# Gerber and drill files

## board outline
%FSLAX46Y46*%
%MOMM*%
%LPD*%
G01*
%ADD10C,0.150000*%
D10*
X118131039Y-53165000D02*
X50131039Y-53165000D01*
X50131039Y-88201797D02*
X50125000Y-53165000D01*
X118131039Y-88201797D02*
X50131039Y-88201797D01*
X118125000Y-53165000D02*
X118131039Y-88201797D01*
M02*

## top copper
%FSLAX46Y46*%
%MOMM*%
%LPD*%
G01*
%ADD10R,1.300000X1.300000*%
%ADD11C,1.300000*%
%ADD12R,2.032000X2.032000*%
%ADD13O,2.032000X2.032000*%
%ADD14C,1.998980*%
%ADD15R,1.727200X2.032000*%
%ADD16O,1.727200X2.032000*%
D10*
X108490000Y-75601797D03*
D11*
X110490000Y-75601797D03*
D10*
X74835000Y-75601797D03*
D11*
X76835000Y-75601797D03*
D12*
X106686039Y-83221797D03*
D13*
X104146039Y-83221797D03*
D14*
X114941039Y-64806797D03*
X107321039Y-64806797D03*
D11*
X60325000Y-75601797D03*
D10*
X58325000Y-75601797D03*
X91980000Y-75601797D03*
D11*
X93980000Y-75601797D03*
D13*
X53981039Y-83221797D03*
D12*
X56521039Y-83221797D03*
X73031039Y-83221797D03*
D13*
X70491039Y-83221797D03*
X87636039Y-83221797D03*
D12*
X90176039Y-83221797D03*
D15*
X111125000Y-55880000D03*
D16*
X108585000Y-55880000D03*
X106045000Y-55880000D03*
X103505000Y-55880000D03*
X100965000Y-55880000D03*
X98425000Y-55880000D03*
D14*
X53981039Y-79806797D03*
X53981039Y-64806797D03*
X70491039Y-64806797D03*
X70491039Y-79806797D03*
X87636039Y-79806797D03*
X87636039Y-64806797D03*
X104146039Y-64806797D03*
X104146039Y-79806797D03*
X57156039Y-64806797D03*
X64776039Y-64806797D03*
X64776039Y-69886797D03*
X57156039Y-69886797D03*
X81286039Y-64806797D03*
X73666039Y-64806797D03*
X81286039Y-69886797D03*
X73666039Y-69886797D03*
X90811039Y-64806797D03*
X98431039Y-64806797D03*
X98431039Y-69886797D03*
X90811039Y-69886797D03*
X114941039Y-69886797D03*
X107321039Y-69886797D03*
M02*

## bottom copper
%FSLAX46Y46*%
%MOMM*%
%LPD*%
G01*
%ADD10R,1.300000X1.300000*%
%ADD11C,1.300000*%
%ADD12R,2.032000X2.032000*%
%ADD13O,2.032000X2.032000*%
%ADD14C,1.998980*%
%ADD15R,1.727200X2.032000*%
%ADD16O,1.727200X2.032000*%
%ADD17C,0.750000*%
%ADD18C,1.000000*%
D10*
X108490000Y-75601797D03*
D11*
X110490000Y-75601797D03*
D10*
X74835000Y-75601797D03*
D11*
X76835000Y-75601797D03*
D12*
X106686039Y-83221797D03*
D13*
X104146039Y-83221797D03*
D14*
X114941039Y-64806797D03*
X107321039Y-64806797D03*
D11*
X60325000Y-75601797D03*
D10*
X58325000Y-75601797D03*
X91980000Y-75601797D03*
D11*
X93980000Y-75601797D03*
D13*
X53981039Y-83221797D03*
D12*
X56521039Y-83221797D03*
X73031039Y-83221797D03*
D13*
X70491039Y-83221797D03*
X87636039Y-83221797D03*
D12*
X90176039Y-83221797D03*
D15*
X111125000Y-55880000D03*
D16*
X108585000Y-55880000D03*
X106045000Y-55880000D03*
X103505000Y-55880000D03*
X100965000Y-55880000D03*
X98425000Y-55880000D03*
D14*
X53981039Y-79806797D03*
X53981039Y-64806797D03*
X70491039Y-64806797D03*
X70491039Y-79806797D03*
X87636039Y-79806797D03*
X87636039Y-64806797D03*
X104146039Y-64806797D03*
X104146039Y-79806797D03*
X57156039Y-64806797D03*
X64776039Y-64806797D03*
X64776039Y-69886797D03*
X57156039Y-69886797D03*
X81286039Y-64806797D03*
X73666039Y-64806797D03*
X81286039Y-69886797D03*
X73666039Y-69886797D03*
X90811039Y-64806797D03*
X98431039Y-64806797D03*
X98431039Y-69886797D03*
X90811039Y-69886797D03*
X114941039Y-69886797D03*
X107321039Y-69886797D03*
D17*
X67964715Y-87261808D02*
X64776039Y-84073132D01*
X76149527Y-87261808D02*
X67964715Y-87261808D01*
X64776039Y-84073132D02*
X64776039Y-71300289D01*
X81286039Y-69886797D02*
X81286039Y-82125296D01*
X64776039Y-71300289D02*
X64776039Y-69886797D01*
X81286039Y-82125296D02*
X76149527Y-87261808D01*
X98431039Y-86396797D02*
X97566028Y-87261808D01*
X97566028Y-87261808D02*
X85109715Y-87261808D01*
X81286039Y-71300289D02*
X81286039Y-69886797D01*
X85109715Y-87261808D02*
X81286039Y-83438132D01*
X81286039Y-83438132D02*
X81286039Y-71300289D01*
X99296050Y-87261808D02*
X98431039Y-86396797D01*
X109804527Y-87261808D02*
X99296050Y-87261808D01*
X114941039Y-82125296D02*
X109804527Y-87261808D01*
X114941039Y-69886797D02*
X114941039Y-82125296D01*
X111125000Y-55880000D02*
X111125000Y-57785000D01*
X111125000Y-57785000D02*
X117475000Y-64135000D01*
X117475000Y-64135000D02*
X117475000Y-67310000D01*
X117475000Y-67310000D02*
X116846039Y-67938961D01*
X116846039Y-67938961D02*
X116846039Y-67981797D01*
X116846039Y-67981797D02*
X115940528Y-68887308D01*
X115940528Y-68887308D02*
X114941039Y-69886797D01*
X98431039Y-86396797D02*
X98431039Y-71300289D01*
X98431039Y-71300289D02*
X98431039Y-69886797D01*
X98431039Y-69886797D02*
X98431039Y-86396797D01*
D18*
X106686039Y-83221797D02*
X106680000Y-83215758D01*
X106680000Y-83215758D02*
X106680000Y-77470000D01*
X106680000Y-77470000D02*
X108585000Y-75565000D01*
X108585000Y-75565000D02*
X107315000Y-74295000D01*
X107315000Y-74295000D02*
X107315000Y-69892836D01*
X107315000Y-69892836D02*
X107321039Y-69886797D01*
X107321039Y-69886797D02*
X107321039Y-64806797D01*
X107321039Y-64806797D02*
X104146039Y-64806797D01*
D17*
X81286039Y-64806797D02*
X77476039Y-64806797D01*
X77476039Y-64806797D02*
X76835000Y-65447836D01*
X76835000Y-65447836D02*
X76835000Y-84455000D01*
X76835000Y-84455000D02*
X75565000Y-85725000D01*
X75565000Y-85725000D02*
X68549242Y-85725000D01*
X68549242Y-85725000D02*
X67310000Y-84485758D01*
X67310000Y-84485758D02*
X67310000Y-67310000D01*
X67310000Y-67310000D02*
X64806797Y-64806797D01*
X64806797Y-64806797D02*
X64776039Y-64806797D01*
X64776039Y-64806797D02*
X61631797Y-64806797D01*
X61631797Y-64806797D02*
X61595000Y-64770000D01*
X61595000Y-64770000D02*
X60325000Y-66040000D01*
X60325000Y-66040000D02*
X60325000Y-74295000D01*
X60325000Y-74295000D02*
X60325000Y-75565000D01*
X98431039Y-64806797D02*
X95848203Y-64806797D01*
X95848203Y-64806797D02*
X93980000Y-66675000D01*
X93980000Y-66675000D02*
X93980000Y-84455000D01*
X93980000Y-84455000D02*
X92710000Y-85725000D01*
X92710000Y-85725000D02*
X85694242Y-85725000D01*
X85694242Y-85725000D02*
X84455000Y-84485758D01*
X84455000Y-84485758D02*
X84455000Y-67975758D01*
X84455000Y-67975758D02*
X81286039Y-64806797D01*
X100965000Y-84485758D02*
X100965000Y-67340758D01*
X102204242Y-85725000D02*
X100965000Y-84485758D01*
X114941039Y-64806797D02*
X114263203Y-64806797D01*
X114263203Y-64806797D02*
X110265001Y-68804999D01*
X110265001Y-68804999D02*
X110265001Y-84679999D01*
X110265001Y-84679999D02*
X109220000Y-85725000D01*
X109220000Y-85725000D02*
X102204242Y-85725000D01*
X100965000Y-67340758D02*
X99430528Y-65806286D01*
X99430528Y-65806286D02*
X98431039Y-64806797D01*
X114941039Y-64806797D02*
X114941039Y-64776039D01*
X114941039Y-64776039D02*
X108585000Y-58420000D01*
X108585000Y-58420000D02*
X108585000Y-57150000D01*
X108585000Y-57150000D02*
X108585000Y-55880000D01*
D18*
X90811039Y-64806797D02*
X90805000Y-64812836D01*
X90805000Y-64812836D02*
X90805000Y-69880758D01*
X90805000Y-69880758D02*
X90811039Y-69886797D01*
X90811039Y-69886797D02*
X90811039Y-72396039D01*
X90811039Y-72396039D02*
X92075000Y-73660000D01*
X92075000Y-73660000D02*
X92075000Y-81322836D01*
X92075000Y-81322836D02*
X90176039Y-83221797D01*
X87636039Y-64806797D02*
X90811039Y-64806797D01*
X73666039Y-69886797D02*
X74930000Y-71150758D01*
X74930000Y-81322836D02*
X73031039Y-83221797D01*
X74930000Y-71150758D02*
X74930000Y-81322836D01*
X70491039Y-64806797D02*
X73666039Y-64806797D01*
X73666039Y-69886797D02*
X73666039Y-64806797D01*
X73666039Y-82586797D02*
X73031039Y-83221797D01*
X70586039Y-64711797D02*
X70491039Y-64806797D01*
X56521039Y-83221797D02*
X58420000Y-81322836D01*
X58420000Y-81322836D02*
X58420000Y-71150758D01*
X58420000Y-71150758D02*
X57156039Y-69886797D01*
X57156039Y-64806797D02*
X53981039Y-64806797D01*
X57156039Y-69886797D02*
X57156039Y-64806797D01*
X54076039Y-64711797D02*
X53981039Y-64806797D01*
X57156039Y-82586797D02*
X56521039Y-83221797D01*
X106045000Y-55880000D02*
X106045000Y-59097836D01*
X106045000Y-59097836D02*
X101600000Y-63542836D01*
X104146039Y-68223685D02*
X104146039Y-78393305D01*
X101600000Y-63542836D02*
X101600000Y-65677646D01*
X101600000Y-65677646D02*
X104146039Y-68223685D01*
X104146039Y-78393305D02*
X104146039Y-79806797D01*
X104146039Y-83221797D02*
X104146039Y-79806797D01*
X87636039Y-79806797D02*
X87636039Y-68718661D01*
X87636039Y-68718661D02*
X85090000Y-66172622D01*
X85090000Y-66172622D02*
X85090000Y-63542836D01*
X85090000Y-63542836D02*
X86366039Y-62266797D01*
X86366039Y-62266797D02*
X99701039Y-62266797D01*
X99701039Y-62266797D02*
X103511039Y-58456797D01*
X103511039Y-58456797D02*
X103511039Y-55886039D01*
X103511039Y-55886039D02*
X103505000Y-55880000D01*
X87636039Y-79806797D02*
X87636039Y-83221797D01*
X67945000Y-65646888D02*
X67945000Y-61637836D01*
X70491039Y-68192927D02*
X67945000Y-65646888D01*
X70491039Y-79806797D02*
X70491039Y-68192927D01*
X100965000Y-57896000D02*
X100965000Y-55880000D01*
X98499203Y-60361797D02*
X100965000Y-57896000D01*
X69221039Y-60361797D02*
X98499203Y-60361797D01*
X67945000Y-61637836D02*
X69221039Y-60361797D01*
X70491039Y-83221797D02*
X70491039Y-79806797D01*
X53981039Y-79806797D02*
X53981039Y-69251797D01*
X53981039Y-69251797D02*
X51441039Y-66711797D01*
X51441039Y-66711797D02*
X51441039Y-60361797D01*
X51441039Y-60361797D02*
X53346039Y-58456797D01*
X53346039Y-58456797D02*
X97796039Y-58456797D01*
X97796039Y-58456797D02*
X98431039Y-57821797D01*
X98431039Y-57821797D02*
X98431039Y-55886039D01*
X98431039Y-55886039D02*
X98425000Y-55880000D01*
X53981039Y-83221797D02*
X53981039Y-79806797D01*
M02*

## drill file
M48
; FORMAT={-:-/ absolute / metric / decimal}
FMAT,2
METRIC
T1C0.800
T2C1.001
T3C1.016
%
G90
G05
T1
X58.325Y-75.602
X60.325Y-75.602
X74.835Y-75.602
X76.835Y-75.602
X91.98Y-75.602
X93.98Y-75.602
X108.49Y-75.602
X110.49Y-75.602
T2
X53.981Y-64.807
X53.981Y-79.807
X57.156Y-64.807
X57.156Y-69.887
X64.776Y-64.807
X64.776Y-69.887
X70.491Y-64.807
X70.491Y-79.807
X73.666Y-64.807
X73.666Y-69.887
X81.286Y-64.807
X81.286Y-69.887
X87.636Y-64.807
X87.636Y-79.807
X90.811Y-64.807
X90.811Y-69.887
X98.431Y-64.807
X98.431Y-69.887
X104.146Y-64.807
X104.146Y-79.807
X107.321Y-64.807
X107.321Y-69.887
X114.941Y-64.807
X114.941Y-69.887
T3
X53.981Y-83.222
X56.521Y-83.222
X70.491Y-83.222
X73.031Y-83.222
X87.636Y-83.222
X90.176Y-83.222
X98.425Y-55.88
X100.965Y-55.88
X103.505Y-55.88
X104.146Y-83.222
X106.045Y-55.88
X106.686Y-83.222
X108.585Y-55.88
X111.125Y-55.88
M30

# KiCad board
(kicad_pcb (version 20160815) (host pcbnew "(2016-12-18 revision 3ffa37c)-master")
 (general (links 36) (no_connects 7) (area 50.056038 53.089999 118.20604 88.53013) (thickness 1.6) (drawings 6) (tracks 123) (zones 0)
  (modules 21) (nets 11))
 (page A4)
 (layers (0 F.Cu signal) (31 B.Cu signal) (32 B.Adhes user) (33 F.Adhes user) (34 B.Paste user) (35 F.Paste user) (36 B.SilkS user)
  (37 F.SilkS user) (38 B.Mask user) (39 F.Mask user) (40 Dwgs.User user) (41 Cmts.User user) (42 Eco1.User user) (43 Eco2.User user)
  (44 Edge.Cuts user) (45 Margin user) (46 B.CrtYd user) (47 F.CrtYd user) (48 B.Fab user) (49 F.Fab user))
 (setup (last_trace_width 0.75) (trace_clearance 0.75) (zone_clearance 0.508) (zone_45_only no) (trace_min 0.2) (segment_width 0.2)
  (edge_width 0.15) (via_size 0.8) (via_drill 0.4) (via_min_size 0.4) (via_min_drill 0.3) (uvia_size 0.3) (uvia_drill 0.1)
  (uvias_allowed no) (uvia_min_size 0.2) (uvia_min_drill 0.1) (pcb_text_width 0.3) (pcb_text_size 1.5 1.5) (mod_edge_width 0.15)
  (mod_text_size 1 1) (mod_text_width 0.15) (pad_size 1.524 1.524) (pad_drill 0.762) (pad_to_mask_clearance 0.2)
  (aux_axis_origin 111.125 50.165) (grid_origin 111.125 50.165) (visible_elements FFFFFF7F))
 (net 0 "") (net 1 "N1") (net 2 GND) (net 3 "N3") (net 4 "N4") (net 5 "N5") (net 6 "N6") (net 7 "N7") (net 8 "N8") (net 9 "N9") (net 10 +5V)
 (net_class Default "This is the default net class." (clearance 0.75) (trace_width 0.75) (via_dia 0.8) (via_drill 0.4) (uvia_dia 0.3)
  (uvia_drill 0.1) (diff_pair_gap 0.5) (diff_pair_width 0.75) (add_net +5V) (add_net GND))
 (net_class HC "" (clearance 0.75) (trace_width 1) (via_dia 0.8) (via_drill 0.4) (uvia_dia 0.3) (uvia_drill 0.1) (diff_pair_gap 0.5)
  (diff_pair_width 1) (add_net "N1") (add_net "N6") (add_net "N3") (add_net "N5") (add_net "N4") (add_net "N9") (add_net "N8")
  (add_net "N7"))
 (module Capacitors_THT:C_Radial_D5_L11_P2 (layer F.Cu) (at 108.49 75.601797)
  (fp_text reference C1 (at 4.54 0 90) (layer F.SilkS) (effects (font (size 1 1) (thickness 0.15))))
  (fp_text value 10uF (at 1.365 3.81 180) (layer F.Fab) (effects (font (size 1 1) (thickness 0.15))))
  (pad 1 thru_hole rect (at 0 0) (size 1.3 1.3) (drill 0.8) (layers *.Cu *.Mask) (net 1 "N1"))
  (pad 2 thru_hole circle (at 2 0) (size 1.3 1.3) (drill 0.8) (layers *.Cu *.Mask) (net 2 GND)))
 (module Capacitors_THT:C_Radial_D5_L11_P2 (layer F.Cu) (at 74.835 75.601797)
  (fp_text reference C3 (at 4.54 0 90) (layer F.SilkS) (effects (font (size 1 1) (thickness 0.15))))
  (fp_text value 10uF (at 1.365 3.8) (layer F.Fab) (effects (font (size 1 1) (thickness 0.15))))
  (pad 1 thru_hole rect (at 0 0) (size 1.3 1.3) (drill 0.8) (layers *.Cu *.Mask) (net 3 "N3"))
  (pad 2 thru_hole circle (at 2 0) (size 1.3 1.3) (drill 0.8) (layers *.Cu *.Mask) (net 2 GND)))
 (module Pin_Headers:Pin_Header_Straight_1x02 (layer F.Cu) (at 106.686039 83.221797 270)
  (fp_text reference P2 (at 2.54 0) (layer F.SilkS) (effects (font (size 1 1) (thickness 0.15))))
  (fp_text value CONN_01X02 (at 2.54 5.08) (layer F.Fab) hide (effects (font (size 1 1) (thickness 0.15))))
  (pad 1 thru_hole rect (at 0 0 270) (size 2.032 2.032) (drill 1.016) (layers *.Cu *.Mask) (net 1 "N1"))
  (pad 2 thru_hole oval (at 0 2.54 270) (size 2.032 2.032) (drill 1.016) (layers *.Cu *.Mask) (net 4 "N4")))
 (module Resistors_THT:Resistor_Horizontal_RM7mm (layer F.Cu) (at 107.321039 64.806797)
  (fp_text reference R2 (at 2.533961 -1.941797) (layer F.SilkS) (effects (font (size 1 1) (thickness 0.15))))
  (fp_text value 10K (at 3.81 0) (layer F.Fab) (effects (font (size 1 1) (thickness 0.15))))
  (pad 2 thru_hole circle (at 7.62 0) (size 1.99898 1.99898) (drill 1.00076) (layers *.Cu *.SilkS *.Mask) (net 2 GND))
  (pad 1 thru_hole circle (at 0 0) (size 1.99898 1.99898) (drill 1.00076) (layers *.Cu *.SilkS *.Mask) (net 1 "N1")))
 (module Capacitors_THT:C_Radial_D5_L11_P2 (layer F.Cu) (at 58.325 75.601797)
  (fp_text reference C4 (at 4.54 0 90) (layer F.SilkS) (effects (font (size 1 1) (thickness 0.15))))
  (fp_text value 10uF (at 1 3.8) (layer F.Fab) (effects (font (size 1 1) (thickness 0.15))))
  (pad 2 thru_hole circle (at 2 0) (size 1.3 1.3) (drill 0.8) (layers *.Cu *.Mask) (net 2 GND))
  (pad 1 thru_hole rect (at 0 0) (size 1.3 1.3) (drill 0.8) (layers *.Cu *.Mask) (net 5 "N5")))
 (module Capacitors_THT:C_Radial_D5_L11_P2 (layer F.Cu) (at 91.98 75.601797)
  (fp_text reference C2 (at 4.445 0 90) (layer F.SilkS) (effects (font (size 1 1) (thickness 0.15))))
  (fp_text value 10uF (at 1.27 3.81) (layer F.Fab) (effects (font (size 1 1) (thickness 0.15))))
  (pad 1 thru_hole rect (at 0 0) (size 1.3 1.3) (drill 0.8) (layers *.Cu *.Mask) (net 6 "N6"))
  (pad 2 thru_hole circle (at 2 0) (size 1.3 1.3) (drill 0.8) (layers *.Cu *.Mask) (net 2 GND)))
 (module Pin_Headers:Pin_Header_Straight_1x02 (layer F.Cu) (at 56.521039 83.221797 270)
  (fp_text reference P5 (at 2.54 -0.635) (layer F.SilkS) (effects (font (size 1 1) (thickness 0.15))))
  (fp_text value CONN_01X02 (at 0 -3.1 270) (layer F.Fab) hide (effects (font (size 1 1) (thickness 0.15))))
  (pad 2 thru_hole oval (at 0 2.54 270) (size 2.032 2.032) (drill 1.016) (layers *.Cu *.Mask) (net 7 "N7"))
  (pad 1 thru_hole rect (at 0 0 270) (size 2.032 2.032) (drill 1.016) (layers *.Cu *.Mask) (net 5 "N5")))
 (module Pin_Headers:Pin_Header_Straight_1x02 (layer F.Cu) (at 73.031039 83.221797 270)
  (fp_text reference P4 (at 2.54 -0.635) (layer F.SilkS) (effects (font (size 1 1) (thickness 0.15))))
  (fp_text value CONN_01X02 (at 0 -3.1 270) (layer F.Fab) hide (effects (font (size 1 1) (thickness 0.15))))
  (pad 1 thru_hole rect (at 0 0 270) (size 2.032 2.032) (drill 1.016) (layers *.Cu *.Mask) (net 3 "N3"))
  (pad 2 thru_hole oval (at 0 2.54 270) (size 2.032 2.032) (drill 1.016) (layers *.Cu *.Mask) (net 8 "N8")))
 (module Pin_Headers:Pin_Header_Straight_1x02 (layer F.Cu) (at 90.176039 83.221797 270)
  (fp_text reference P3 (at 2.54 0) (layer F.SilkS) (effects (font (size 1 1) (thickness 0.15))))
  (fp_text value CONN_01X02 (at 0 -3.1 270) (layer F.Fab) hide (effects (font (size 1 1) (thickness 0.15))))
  (pad 2 thru_hole oval (at 0 2.54 270) (size 2.032 2.032) (drill 1.016) (layers *.Cu *.Mask) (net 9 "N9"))
  (pad 1 thru_hole rect (at 0 0 270) (size 2.032 2.032) (drill 1.016) (layers *.Cu *.Mask) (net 6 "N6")))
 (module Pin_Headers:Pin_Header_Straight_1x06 (layer F.Cu) (at 111.125 55.88 270)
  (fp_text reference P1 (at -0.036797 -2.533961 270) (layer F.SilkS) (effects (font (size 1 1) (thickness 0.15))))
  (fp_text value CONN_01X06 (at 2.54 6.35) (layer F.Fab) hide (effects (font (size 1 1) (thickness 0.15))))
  (pad 1 thru_hole rect (at 0 0 270) (size 2.032 1.7272) (drill 1.016) (layers *.Cu *.Mask) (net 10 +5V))
  (pad 2 thru_hole oval (at 0 2.54 270) (size 2.032 1.7272) (drill 1.016) (layers *.Cu *.Mask) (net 2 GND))
  (pad 3 thru_hole oval (at 0 5.08 270) (size 2.032 1.7272) (drill 1.016) (layers *.Cu *.Mask) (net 4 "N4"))
  (pad 4 thru_hole oval (at 0 7.62 270) (size 2.032 1.7272) (drill 1.016) (layers *.Cu *.Mask) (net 9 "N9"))
  (pad 5 thru_hole oval (at 0 10.16 270) (size 2.032 1.7272) (drill 1.016) (layers *.Cu *.Mask) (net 8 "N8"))
  (pad 6 thru_hole oval (at 0 12.7 270) (size 2.032 1.7272) (drill 1.016) (layers *.Cu *.Mask) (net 7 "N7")))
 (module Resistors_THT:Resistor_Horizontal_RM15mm (layer F.Cu) (at 53.981039 64.806797 270)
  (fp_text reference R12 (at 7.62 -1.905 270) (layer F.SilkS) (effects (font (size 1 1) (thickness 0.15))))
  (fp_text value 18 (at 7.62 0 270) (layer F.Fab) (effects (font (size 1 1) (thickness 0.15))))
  (pad 2 thru_hole circle (at 15 0 270) (size 1.99898 1.99898) (drill 1.00076) (layers *.Cu *.SilkS *.Mask) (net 7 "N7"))
  (pad 1 thru_hole circle (at 0 0 270) (size 1.99898 1.99898) (drill 1.00076) (layers *.Cu *.SilkS *.Mask) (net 5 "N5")))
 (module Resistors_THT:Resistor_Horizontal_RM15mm (layer F.Cu) (at 70.491039 64.806797 270)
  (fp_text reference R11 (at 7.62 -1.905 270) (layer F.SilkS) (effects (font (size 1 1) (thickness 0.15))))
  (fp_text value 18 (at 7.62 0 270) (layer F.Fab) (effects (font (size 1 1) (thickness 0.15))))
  (pad 1 thru_hole circle (at 0 0 270) (size 1.99898 1.99898) (drill 1.00076) (layers *.Cu *.SilkS *.Mask) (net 3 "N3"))
  (pad 2 thru_hole circle (at 15 0 270) (size 1.99898 1.99898) (drill 1.00076) (layers *.Cu *.SilkS *.Mask) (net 8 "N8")))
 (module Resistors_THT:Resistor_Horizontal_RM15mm (layer F.Cu) (at 87.636039 64.806797 270)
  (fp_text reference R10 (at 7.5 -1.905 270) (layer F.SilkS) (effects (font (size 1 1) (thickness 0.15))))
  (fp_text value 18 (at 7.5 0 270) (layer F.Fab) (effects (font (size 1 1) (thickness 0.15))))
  (pad 2 thru_hole circle (at 15 0 270) (size 1.99898 1.99898) (drill 1.00076) (layers *.Cu *.SilkS *.Mask) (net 9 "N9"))
  (pad 1 thru_hole circle (at 0 0 270) (size 1.99898 1.99898) (drill 1.00076) (layers *.Cu *.SilkS *.Mask) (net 6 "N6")))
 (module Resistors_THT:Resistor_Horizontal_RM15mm (layer F.Cu) (at 104.146039 64.806797 270)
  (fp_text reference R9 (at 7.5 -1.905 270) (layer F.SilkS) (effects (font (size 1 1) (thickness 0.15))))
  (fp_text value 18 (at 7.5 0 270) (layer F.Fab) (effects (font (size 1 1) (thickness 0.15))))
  (pad 1 thru_hole circle (at 0 0 270) (size 1.99898 1.99898) (drill 1.00076) (layers *.Cu *.SilkS *.Mask) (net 1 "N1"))
  (pad 2 thru_hole circle (at 15 0 270) (size 1.99898 1.99898) (drill 1.00076) (layers *.Cu *.SilkS *.Mask) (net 4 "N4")))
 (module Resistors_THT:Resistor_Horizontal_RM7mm (layer F.Cu) (at 57.156039 64.806797)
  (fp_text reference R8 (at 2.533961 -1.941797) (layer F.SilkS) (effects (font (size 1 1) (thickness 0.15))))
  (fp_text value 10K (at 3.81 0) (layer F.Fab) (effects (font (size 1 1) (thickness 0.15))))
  (pad 1 thru_hole circle (at 0 0) (size 1.99898 1.99898) (drill 1.00076) (layers *.Cu *.SilkS *.Mask) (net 5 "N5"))
  (pad 2 thru_hole circle (at 7.62 0) (size 1.99898 1.99898) (drill 1.00076) (layers *.Cu *.SilkS *.Mask) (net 2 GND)))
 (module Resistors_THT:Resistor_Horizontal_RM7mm (layer F.Cu) (at 64.776039 69.886797 180)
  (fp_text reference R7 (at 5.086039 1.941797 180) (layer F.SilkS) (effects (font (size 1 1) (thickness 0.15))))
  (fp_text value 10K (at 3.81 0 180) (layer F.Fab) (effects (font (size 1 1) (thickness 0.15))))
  (pad 1 thru_hole circle (at 0 0 180) (size 1.99898 1.99898) (drill 1.00076) (layers *.Cu *.SilkS *.Mask) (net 10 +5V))
  (pad 2 thru_hole circle (at 7.62 0 180) (size 1.99898 1.99898) (drill 1.00076) (layers *.Cu *.SilkS *.Mask) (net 5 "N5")))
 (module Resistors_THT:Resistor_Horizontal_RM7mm (layer F.Cu) (at 73.666039 64.806797)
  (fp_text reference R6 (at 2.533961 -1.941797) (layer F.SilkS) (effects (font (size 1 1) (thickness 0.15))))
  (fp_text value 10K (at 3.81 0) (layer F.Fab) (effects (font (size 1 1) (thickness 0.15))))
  (pad 2 thru_hole circle (at 7.62 0) (size 1.99898 1.99898) (drill 1.00076) (layers *.Cu *.SilkS *.Mask) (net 2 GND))
  (pad 1 thru_hole circle (at 0 0) (size 1.99898 1.99898) (drill 1.00076) (layers *.Cu *.SilkS *.Mask) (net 3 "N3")))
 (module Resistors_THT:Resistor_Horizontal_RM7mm (layer F.Cu) (at 81.286039 69.886797 180)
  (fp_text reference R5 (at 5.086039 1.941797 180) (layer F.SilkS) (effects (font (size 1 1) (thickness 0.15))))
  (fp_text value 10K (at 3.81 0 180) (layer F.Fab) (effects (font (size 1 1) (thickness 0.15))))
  (pad 1 thru_hole circle (at 0 0 180) (size 1.99898 1.99898) (drill 1.00076) (layers *.Cu *.SilkS *.Mask) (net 10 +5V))
  (pad 2 thru_hole circle (at 7.62 0 180) (size 1.99898 1.99898) (drill 1.00076) (layers *.Cu *.SilkS *.Mask) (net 3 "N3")))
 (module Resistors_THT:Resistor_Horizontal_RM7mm (layer F.Cu) (at 90.811039 64.806797)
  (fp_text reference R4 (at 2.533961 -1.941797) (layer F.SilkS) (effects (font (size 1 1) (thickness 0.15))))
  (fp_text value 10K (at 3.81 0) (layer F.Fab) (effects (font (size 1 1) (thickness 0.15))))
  (pad 1 thru_hole circle (at 0 0) (size 1.99898 1.99898) (drill 1.00076) (layers *.Cu *.SilkS *.Mask) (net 6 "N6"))
  (pad 2 thru_hole circle (at 7.62 0) (size 1.99898 1.99898) (drill 1.00076) (layers *.Cu *.SilkS *.Mask) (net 2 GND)))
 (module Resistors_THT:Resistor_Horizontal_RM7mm (layer F.Cu) (at 98.431039 69.886797 180)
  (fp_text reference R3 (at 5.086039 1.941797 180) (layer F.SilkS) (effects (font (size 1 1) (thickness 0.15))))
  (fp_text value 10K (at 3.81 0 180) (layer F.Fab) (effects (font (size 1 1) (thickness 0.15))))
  (pad 1 thru_hole circle (at 0 0 180) (size 1.99898 1.99898) (drill 1.00076) (layers *.Cu *.SilkS *.Mask) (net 10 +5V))
  (pad 2 thru_hole circle (at 7.62 0 180) (size 1.99898 1.99898) (drill 1.00076) (layers *.Cu *.SilkS *.Mask) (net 6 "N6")))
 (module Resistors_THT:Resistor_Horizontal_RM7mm (layer F.Cu) (at 114.941039 69.886797 180)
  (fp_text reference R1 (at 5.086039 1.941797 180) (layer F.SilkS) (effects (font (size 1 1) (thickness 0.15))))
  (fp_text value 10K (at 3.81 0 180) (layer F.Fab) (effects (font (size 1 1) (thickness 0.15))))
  (pad 1 thru_hole circle (at 0 0 180) (size 1.99898 1.99898) (drill 1.00076) (layers *.Cu *.SilkS *.Mask) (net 10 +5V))
  (pad 2 thru_hole circle (at 7.62 0 180) (size 1.99898 1.99898) (drill 1.00076) (layers *.Cu *.SilkS *.Mask) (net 1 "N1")))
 (gr_line (start 118.131039 53.165) (end 50.131039 53.165) (angle 90) (layer Edge.Cuts) (width 0.15))
 (gr_line (start 50.131039 88.201797) (end 50.125 53.165) (angle 90) (layer Edge.Cuts) (width 0.15))
 (gr_line (start 118.131039 88.201797) (end 50.131039 88.201797) (angle 90) (layer Edge.Cuts) (width 0.15))
 (gr_line (start 118.125 53.165) (end 118.131039 88.201797) (angle 90) (layer Edge.Cuts) (width 0.15))
 (segment (start 67.964715 87.261808) (end 64.776039 84.073132) (width 0.75) (layer B.Cu) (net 10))
 (segment (start 76.149527 87.261808) (end 67.964715 87.261808) (width 0.75) (layer B.Cu) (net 10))
 (segment (start 64.776039 84.073132) (end 64.776039 71.300289) (width 0.75) (layer B.Cu) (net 10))
 (segment (start 81.286039 69.886797) (end 81.286039 82.125296) (width 0.75) (layer B.Cu) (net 10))
 (segment (start 64.776039 71.300289) (end 64.776039 69.886797) (width 0.75) (layer B.Cu) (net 10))
 (segment (start 81.286039 82.125296) (end 76.149527 87.261808) (width 0.75) (layer B.Cu) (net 10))
 (segment (start 98.431039 86.396797) (end 97.566028 87.261808) (width 0.75) (layer B.Cu) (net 10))
 (segment (start 97.566028 87.261808) (end 85.109715 87.261808) (width 0.75) (layer B.Cu) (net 10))
 (segment (start 81.286039 71.300289) (end 81.286039 69.886797) (width 0.75) (layer B.Cu) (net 10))
 (segment (start 85.109715 87.261808) (end 81.286039 83.438132) (width 0.75) (layer B.Cu) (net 10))
 (segment (start 81.286039 83.438132) (end 81.286039 71.300289) (width 0.75) (layer B.Cu) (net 10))
 (segment (start 99.29605 87.261808) (end 98.431039 86.396797) (width 0.75) (layer B.Cu) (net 10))
 (segment (start 109.804527 87.261808) (end 99.29605 87.261808) (width 0.75) (layer B.Cu) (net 10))
 (segment (start 114.941039 82.125296) (end 109.804527 87.261808) (width 0.75) (layer B.Cu) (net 10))
 (segment (start 114.941039 69.886797) (end 114.941039 82.125296) (width 0.75) (layer B.Cu) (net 10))
 (segment (start 111.125 55.88) (end 111.125 57.785) (width 0.75) (layer B.Cu) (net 10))
 (segment (start 111.125 57.785) (end 117.475 64.135) (width 0.75) (layer B.Cu) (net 10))
 (segment (start 117.475 64.135) (end 117.475 67.31) (width 0.75) (layer B.Cu) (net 10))
 (segment (start 117.475 67.31) (end 116.846039 67.938961) (width 0.75) (layer B.Cu) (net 10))
 (segment (start 116.846039 67.938961) (end 116.846039 67.981797) (width 0.75) (layer B.Cu) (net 10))
 (segment (start 116.846039 67.981797) (end 115.940528 68.887308) (width 0.75) (layer B.Cu) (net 10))
 (segment (start 115.940528 68.887308) (end 114.941039 69.886797) (width 0.75) (layer B.Cu) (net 10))
 (segment (start 98.431039 86.396797) (end 98.431039 71.300289) (width 0.75) (layer B.Cu) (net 10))
 (segment (start 98.431039 71.300289) (end 98.431039 69.886797) (width 0.75) (layer B.Cu) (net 10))
 (segment (start 98.431039 69.886797) (end 98.431039 86.396797) (width 0.75) (layer B.Cu) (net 10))
 (segment (start 106.686039 83.221797) (end 106.68 83.215758) (width 1) (layer B.Cu) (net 1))
 (segment (start 106.68 83.215758) (end 106.68 77.47) (width 1) (layer B.Cu) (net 1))
 (segment (start 106.68 77.47) (end 108.585 75.565) (width 1) (layer B.Cu) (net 1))
 (segment (start 108.585 75.565) (end 107.315 74.295) (width 1) (layer B.Cu) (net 1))
 (segment (start 107.315 74.295) (end 107.315 69.892836) (width 1) (layer B.Cu) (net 1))
 (segment (start 107.315 69.892836) (end 107.321039 69.886797) (width 1) (layer B.Cu) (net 1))
 (segment (start 107.321039 69.886797) (end 107.321039 64.806797) (width 1) (layer B.Cu) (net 1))
 (segment (start 107.321039 64.806797) (end 104.146039 64.806797) (width 1) (layer B.Cu) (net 1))
 (segment (start 81.286039 64.806797) (end 77.476039 64.806797) (width 0.75) (layer B.Cu) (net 2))
 (segment (start 77.476039 64.806797) (end 76.835 65.447836) (width 0.75) (layer B.Cu) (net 2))
 (segment (start 76.835 65.447836) (end 76.835 84.455) (width 0.75) (layer B.Cu) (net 2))
 (segment (start 76.835 84.455) (end 75.565 85.725) (width 0.75) (layer B.Cu) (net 2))
 (segment (start 75.565 85.725) (end 68.549242 85.725) (width 0.75) (layer B.Cu) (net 2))
 (segment (start 68.549242 85.725) (end 67.31 84.485758) (width 0.75) (layer B.Cu) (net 2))
 (segment (start 67.31 84.485758) (end 67.31 67.31) (width 0.75) (layer B.Cu) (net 2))
 (segment (start 67.31 67.31) (end 64.806797 64.806797) (width 0.75) (layer B.Cu) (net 2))
 (segment (start 64.806797 64.806797) (end 64.776039 64.806797) (width 0.75) (layer B.Cu) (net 2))
 (segment (start 64.776039 64.806797) (end 61.631797 64.806797) (width 0.75) (layer B.Cu) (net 2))
 (segment (start 61.631797 64.806797) (end 61.595 64.77) (width 0.75) (layer B.Cu) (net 2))
 (segment (start 61.595 64.77) (end 60.325 66.04) (width 0.75) (layer B.Cu) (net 2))
 (segment (start 60.325 66.04) (end 60.325 74.295) (width 0.75) (layer B.Cu) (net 2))
 (segment (start 60.325 74.295) (end 60.325 75.565) (width 0.75) (layer B.Cu) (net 2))
 (segment (start 98.431039 64.806797) (end 95.848203 64.806797) (width 0.75) (layer B.Cu) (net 2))
 (segment (start 95.848203 64.806797) (end 93.98 66.675) (width 0.75) (layer B.Cu) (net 2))
 (segment (start 93.98 66.675) (end 93.98 84.455) (width 0.75) (layer B.Cu) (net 2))
 (segment (start 93.98 84.455) (end 92.71 85.725) (width 0.75) (layer B.Cu) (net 2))
 (segment (start 92.71 85.725) (end 85.694242 85.725) (width 0.75) (layer B.Cu) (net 2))
 (segment (start 85.694242 85.725) (end 84.455 84.485758) (width 0.75) (layer B.Cu) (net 2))
 (segment (start 84.455 84.485758) (end 84.455 67.975758) (width 0.75) (layer B.Cu) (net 2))
 (segment (start 84.455 67.975758) (end 81.286039 64.806797) (width 0.75) (layer B.Cu) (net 2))
 (segment (start 100.965 84.485758) (end 100.965 67.340758) (width 0.75) (layer B.Cu) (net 2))
 (segment (start 102.204242 85.725) (end 100.965 84.485758) (width 0.75) (layer B.Cu) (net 2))
 (segment (start 114.941039 64.806797) (end 114.263203 64.806797) (width 0.75) (layer B.Cu) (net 2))
 (segment (start 114.263203 64.806797) (end 110.265001 68.804999) (width 0.75) (layer B.Cu) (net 2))
 (segment (start 110.265001 68.804999) (end 110.265001 84.679999) (width 0.75) (layer B.Cu) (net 2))
 (segment (start 110.265001 84.679999) (end 109.22 85.725) (width 0.75) (layer B.Cu) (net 2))
 (segment (start 109.22 85.725) (end 102.204242 85.725) (width 0.75) (layer B.Cu) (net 2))
 (segment (start 100.965 67.340758) (end 99.430528 65.806286) (width 0.75) (layer B.Cu) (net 2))
 (segment (start 99.430528 65.806286) (end 98.431039 64.806797) (width 0.75) (layer B.Cu) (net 2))
 (segment (start 114.941039 64.806797) (end 114.941039 64.776039) (width 0.75) (layer B.Cu) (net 2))
 (segment (start 114.941039 64.776039) (end 108.585 58.42) (width 0.75) (layer B.Cu) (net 2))
 (segment (start 108.585 58.42) (end 108.585 57.15) (width 0.75) (layer B.Cu) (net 2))
 (segment (start 108.585 57.15) (end 108.585 55.88) (width 0.75) (layer B.Cu) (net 2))
 (segment (start 90.811039 64.806797) (end 90.805 64.812836) (width 1) (layer B.Cu) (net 6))
 (segment (start 90.805 64.812836) (end 90.805 69.880758) (width 1) (layer B.Cu) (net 6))
 (segment (start 90.805 69.880758) (end 90.811039 69.886797) (width 1) (layer B.Cu) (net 6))
 (segment (start 90.811039 69.886797) (end 90.811039 72.396039) (width 1) (layer B.Cu) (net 6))
 (segment (start 90.811039 72.396039) (end 92.075 73.66) (width 1) (layer B.Cu) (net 6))
 (segment (start 92.075 73.66) (end 92.075 81.322836) (width 1) (layer B.Cu) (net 6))
 (segment (start 92.075 81.322836) (end 90.176039 83.221797) (width 1) (layer B.Cu) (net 6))
 (segment (start 87.636039 64.806797) (end 90.811039 64.806797) (width 1) (layer B.Cu) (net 6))
 (segment (start 73.666039 69.886797) (end 74.93 71.150758) (width 1) (layer B.Cu) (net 3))
 (segment (start 74.93 81.322836) (end 73.031039 83.221797) (width 1) (layer B.Cu) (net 3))
 (segment (start 74.93 71.150758) (end 74.93 81.322836) (width 1) (layer B.Cu) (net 3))
 (segment (start 70.491039 64.806797) (end 73.666039 64.806797) (width 1) (layer B.Cu) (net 3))
 (segment (start 73.666039 69.886797) (end 73.666039 64.806797) (width 1) (layer B.Cu) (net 3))
 (segment (start 73.666039 82.586797) (end 73.031039 83.221797) (width 1) (layer B.Cu) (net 3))
 (segment (start 70.586039 64.711797) (end 70.491039 64.806797) (width 1) (layer B.Cu) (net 3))
 (segment (start 56.521039 83.221797) (end 58.42 81.322836) (width 1) (layer B.Cu) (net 5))
 (segment (start 58.42 81.322836) (end 58.42 71.150758) (width 1) (layer B.Cu) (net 5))
 (segment (start 58.42 71.150758) (end 57.156039 69.886797) (width 1) (layer B.Cu) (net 5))
 (segment (start 57.156039 64.806797) (end 53.981039 64.806797) (width 1) (layer B.Cu) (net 5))
 (segment (start 57.156039 69.886797) (end 57.156039 64.806797) (width 1) (layer B.Cu) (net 5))
 (segment (start 54.076039 64.711797) (end 53.981039 64.806797) (width 1) (layer B.Cu) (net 5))
 (segment (start 57.156039 82.586797) (end 56.521039 83.221797) (width 1) (layer B.Cu) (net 5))
 (segment (start 106.045 55.88) (end 106.045 59.097836) (width 1) (layer B.Cu) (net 4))
 (segment (start 106.045 59.097836) (end 101.6 63.542836) (width 1) (layer B.Cu) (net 4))
 (segment (start 104.146039 68.223685) (end 104.146039 78.393305) (width 1) (layer B.Cu) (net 4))
 (segment (start 101.6 63.542836) (end 101.6 65.677646) (width 1) (layer B.Cu) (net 4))
 (segment (start 101.6 65.677646) (end 104.146039 68.223685) (width 1) (layer B.Cu) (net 4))
 (segment (start 104.146039 78.393305) (end 104.146039 79.806797) (width 1) (layer B.Cu) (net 4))
 (segment (start 104.146039 83.221797) (end 104.146039 79.806797) (width 1) (layer B.Cu) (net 4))
 (segment (start 87.636039 79.806797) (end 87.636039 68.718661) (width 1) (layer B.Cu) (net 9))
 (segment (start 87.636039 68.718661) (end 85.09 66.172622) (width 1) (layer B.Cu) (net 9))
 (segment (start 85.09 66.172622) (end 85.09 63.542836) (width 1) (layer B.Cu) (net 9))
 (segment (start 85.09 63.542836) (end 86.366039 62.266797) (width 1) (layer B.Cu) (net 9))
 (segment (start 86.366039 62.266797) (end 99.701039 62.266797) (width 1) (layer B.Cu) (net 9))
 (segment (start 99.701039 62.266797) (end 103.511039 58.456797) (width 1) (layer B.Cu) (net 9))
 (segment (start 103.511039 58.456797) (end 103.511039 55.886039) (width 1) (layer B.Cu) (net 9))
 (segment (start 103.511039 55.886039) (end 103.505 55.88) (width 1) (layer B.Cu) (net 9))
 (segment (start 87.636039 79.806797) (end 87.636039 83.221797) (width 1) (layer B.Cu) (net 9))
 (segment (start 67.945 65.646888) (end 67.945 61.637836) (width 1) (layer B.Cu) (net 8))
 (segment (start 70.491039 68.192927) (end 67.945 65.646888) (width 1) (layer B.Cu) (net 8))
 (segment (start 70.491039 79.806797) (end 70.491039 68.192927) (width 1) (layer B.Cu) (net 8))
 (segment (start 100.965 57.896) (end 100.965 55.88) (width 1) (layer B.Cu) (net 8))
 (segment (start 98.499203 60.361797) (end 100.965 57.896) (width 1) (layer B.Cu) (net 8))
 (segment (start 69.221039 60.361797) (end 98.499203 60.361797) (width 1) (layer B.Cu) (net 8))
 (segment (start 67.945 61.637836) (end 69.221039 60.361797) (width 1) (layer B.Cu) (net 8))
 (segment (start 70.491039 83.221797) (end 70.491039 79.806797) (width 1) (layer B.Cu) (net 8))
 (segment (start 53.981039 79.806797) (end 53.981039 69.251797) (width 1) (layer B.Cu) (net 7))
 (segment (start 53.981039 69.251797) (end 51.441039 66.711797) (width 1) (layer B.Cu) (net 7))
 (segment (start 51.441039 66.711797) (end 51.441039 60.361797) (width 1) (layer B.Cu) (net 7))
 (segment (start 51.441039 60.361797) (end 53.346039 58.456797) (width 1) (layer B.Cu) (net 7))
 (segment (start 53.346039 58.456797) (end 97.796039 58.456797) (width 1) (layer B.Cu) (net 7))
 (segment (start 97.796039 58.456797) (end 98.431039 57.821797) (width 1) (layer B.Cu) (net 7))
 (segment (start 98.431039 57.821797) (end 98.431039 55.886039) (width 1) (layer B.Cu) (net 7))
 (segment (start 98.431039 55.886039) (end 98.425 55.88) (width 1) (layer B.Cu) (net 7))
 (segment (start 53.981039 83.221797) (end 53.981039 79.806797) (width 1) (layer B.Cu) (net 7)))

